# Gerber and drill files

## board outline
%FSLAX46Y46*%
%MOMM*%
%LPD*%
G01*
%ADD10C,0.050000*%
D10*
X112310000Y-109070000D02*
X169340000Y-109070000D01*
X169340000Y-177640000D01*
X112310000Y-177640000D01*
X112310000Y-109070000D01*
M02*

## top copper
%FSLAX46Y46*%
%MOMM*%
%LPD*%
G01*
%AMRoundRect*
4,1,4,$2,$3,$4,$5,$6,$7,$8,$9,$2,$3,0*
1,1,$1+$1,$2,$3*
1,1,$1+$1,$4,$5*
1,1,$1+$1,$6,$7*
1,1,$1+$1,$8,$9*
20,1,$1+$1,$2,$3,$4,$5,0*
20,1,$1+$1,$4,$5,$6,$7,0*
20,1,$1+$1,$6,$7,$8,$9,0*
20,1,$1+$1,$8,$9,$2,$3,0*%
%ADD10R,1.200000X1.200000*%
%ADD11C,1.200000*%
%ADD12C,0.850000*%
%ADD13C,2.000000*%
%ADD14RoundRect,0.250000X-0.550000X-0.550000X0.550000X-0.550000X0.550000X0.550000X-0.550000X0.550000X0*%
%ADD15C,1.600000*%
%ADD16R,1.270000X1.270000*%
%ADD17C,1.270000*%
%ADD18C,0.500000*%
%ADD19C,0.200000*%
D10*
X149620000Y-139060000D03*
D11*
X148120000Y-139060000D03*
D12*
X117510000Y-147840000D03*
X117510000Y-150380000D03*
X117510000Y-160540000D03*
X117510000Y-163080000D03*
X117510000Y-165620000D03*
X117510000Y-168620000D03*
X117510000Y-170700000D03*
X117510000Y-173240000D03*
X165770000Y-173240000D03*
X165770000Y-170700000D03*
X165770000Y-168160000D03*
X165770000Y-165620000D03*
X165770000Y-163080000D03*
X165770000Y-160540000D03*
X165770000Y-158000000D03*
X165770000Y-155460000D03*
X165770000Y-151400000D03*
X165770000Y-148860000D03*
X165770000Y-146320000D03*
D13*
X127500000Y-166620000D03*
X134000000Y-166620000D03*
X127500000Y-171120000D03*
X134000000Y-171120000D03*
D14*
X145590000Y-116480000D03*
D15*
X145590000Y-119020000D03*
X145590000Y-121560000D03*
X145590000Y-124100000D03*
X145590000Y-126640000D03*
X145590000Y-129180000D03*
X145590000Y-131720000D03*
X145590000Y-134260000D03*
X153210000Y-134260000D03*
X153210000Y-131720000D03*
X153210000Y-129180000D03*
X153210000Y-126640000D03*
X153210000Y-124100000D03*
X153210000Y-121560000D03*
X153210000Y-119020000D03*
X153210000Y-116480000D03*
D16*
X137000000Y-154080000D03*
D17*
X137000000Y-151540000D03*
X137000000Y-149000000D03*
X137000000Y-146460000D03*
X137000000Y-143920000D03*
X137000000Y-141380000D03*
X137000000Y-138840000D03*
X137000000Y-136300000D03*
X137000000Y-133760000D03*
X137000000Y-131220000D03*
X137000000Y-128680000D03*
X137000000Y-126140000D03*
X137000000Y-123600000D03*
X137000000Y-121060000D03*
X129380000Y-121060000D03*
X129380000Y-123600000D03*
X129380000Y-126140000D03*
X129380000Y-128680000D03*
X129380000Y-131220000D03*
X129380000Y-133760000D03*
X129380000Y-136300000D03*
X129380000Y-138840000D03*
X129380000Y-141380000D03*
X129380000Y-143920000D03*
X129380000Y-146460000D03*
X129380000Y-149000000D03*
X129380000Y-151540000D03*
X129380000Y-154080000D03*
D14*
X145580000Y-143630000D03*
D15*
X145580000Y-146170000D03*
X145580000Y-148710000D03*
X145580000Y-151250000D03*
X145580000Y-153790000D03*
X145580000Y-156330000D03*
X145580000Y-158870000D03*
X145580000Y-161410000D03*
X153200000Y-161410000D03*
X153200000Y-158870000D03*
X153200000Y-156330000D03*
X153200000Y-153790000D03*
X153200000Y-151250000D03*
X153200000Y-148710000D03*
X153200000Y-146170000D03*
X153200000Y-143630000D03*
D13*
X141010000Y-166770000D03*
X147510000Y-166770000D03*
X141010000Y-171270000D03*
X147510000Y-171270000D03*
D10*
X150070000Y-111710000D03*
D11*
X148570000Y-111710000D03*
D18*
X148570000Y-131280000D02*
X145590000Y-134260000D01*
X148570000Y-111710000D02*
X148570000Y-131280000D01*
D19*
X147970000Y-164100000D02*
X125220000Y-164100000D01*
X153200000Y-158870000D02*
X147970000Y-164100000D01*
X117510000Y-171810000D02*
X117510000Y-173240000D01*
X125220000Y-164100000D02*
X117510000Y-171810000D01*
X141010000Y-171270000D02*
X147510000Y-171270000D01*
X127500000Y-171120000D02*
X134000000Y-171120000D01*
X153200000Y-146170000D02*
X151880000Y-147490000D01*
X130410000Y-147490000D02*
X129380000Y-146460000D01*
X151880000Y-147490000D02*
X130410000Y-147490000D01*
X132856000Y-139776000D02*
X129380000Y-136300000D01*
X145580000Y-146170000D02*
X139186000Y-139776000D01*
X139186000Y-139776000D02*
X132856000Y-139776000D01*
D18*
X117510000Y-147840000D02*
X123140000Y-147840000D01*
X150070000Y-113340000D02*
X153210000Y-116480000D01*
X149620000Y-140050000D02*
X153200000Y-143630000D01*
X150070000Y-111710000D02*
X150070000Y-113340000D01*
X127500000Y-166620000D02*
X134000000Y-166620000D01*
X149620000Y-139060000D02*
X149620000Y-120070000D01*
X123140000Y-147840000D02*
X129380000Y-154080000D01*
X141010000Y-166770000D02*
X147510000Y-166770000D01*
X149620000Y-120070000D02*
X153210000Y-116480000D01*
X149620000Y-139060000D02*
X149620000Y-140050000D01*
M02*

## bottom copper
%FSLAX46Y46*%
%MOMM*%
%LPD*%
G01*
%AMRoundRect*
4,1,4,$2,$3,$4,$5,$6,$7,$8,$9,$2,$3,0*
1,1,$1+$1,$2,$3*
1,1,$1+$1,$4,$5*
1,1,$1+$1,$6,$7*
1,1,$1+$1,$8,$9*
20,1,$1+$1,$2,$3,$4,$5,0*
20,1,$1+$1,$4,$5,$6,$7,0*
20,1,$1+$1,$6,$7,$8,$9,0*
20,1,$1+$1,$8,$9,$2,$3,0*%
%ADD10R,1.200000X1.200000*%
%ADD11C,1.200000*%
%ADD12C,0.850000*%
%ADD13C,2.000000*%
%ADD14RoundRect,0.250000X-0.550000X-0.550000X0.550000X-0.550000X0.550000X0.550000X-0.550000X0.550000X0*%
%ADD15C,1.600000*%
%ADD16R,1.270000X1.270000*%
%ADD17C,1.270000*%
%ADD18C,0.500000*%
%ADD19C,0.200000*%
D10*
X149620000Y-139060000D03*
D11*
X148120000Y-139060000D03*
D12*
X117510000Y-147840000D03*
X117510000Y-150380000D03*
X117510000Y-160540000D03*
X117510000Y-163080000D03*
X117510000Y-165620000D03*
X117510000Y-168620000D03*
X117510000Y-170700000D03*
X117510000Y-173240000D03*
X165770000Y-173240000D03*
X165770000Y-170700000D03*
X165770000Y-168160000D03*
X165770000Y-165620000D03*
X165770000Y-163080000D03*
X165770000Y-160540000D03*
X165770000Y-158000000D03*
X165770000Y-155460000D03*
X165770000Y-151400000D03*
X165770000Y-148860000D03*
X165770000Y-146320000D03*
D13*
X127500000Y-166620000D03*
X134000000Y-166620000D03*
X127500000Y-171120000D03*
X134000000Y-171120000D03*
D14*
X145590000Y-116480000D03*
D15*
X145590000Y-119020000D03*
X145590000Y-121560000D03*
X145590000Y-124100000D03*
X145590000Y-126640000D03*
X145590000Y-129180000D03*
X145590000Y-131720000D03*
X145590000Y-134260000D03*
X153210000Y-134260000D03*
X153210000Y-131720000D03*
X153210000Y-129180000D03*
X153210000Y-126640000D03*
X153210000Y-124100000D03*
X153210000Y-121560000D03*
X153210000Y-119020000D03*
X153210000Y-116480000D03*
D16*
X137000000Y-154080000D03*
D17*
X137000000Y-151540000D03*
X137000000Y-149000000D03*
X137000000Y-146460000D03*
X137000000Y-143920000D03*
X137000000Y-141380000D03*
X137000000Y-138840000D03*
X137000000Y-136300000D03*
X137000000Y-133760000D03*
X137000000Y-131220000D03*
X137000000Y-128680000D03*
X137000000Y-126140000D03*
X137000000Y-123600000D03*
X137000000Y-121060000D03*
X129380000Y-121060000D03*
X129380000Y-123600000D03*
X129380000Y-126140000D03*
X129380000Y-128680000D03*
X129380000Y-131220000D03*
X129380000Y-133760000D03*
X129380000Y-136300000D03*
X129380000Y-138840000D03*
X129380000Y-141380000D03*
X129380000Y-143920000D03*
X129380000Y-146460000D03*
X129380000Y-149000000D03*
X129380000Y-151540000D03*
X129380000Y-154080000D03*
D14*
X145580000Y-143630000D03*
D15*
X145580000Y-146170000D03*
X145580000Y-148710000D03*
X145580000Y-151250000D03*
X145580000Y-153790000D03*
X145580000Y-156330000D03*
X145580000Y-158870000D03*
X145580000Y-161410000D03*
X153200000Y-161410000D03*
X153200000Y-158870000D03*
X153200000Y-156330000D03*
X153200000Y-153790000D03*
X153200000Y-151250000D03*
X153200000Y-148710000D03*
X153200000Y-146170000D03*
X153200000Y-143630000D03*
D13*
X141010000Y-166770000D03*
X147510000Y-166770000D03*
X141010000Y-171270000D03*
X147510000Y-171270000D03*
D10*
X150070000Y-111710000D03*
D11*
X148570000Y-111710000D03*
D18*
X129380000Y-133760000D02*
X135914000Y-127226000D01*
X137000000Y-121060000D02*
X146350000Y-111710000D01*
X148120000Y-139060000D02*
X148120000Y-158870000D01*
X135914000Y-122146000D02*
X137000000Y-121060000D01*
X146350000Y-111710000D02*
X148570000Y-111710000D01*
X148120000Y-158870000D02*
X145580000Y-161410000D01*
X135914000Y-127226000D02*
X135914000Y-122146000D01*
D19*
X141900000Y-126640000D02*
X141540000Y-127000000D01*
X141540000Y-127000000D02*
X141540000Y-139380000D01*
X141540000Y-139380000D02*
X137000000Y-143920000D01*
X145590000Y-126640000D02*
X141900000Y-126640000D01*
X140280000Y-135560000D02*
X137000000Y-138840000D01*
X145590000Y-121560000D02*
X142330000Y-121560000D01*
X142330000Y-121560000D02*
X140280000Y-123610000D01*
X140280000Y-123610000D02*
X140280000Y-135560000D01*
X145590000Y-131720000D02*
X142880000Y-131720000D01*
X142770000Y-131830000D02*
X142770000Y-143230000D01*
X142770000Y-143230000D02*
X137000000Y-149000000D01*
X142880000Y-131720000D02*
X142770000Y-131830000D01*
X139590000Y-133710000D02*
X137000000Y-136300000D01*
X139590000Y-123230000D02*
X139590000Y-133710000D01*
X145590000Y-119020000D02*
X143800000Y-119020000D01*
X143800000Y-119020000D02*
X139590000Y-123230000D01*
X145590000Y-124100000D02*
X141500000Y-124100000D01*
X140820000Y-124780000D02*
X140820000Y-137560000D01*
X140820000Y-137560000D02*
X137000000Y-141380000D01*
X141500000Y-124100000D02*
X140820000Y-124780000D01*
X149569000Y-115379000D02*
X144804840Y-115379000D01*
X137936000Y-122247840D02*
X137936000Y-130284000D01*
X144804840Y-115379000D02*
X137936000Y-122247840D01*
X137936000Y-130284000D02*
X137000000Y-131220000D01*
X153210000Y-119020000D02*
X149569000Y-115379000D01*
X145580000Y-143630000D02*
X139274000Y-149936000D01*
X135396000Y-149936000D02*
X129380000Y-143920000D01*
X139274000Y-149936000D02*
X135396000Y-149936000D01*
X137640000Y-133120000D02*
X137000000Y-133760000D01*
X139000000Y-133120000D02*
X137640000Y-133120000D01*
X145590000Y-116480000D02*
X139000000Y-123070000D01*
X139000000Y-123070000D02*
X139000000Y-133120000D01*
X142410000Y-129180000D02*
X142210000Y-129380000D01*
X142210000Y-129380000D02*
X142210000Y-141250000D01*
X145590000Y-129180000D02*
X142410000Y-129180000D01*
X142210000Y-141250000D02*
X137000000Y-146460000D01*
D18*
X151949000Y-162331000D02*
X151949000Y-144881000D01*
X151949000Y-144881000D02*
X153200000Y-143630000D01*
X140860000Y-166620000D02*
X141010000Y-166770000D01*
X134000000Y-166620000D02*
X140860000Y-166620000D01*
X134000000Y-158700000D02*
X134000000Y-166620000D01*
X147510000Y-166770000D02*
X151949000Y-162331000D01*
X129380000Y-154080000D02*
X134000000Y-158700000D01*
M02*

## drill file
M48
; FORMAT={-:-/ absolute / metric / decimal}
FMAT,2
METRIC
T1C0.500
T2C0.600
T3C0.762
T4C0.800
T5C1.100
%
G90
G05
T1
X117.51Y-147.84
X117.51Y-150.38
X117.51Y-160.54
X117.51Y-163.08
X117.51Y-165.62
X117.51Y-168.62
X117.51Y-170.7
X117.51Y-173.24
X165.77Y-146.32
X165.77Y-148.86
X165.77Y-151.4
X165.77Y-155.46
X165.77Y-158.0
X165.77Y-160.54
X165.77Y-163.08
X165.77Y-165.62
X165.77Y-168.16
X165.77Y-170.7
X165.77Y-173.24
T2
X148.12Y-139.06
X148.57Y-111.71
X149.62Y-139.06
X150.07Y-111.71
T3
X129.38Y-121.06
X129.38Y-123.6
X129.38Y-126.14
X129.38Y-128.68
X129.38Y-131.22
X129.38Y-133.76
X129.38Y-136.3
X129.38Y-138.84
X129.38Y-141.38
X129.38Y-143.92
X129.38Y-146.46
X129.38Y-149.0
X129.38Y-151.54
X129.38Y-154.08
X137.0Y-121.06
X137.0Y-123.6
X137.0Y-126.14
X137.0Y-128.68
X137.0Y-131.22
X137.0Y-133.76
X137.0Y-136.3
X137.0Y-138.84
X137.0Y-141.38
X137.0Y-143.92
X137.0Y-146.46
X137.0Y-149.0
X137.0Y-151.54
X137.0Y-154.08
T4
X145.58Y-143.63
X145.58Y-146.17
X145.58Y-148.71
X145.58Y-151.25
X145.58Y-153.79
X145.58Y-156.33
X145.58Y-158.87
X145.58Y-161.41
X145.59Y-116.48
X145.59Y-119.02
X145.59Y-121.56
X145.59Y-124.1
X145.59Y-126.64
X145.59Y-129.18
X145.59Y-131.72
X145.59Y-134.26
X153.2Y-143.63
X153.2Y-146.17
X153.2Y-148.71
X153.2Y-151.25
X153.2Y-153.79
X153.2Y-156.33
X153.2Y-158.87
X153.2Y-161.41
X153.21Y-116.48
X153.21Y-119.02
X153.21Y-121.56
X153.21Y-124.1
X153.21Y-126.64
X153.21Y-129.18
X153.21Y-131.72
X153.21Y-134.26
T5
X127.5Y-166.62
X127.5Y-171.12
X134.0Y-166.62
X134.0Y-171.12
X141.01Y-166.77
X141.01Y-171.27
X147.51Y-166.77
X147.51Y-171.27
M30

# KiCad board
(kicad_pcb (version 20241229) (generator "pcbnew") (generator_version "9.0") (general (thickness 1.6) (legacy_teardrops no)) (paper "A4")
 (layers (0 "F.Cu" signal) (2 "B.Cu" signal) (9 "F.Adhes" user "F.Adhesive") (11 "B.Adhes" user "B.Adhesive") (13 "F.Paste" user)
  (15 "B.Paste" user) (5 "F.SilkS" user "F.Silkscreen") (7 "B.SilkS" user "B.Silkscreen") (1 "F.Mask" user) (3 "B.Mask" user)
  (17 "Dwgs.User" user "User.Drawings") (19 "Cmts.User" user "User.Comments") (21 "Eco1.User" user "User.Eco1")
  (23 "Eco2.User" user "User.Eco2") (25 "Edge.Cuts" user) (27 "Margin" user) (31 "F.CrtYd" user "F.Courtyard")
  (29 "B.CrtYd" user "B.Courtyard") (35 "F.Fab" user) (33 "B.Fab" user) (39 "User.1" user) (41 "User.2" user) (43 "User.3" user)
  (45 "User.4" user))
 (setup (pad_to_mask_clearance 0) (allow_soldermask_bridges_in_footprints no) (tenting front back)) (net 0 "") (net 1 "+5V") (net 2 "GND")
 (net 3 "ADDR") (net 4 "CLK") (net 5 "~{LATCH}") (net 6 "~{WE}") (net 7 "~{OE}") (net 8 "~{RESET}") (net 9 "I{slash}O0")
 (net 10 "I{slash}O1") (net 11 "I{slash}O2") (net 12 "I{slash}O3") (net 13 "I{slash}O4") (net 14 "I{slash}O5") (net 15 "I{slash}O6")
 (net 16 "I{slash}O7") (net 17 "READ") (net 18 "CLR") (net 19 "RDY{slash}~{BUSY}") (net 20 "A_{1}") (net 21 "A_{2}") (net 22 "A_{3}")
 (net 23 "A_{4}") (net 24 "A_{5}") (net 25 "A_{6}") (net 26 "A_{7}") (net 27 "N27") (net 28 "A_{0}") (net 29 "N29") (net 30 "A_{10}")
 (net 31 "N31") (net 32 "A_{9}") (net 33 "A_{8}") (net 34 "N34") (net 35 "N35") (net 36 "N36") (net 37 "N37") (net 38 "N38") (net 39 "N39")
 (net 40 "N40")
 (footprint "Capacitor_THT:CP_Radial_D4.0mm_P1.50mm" (layer "F.Cu") (at 149.62 139.06 180)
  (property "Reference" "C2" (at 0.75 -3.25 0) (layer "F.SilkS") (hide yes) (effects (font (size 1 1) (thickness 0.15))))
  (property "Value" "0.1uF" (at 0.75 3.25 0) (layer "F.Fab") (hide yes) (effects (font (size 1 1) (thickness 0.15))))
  (pad "1" thru_hole rect (at 0 0 180) (size 1.2 1.2) (drill 0.6) (layers "*.Cu" "*.Mask") (remove_unused_layers no) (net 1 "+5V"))
  (pad "2" thru_hole circle (at 1.5 0 180) (size 1.2 1.2) (drill 0.6) (layers "*.Cu" "*.Mask") (remove_unused_layers no) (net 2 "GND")))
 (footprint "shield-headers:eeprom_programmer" (layer "F.Cu") (at 140.37 163.08)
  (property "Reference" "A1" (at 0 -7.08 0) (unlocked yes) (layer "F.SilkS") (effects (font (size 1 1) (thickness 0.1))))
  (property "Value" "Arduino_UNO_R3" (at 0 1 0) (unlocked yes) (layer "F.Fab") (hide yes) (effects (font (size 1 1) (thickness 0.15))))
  (pad "5" thru_hole circle (at -22.86 -15.24) (size 0.85 0.85) (drill 0.5) (layers "*.Cu" "*.Mask") (remove_unused_layers no) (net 1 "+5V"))
  (pad "6" thru_hole circle (at -22.86 -12.7) (size 0.85 0.85) (drill 0.5) (layers "*.Cu" "*.Mask") (remove_unused_layers no) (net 2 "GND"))
  (pad "9" thru_hole circle (at -22.86 -2.54) (size 0.85 0.85) (drill 0.5) (layers "*.Cu" "*.Mask") (remove_unused_layers no) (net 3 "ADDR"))
  (pad "10" thru_hole circle (at -22.86 0) (size 0.85 0.85) (drill 0.5) (layers "*.Cu" "*.Mask") (remove_unused_layers no) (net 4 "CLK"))
  (pad "11" thru_hole circle (at -22.86 2.54) (size 0.85 0.85) (drill 0.5) (layers "*.Cu" "*.Mask") (remove_unused_layers no)
   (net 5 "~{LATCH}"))
  (pad "12" thru_hole circle (at -22.86 5.54) (size 0.85 0.85) (drill 0.5) (layers "*.Cu" "*.Mask") (remove_unused_layers no)
   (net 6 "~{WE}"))
  (pad "13" thru_hole circle (at -22.86 7.62) (size 0.85 0.85) (drill 0.5) (layers "*.Cu" "*.Mask") (remove_unused_layers no)
   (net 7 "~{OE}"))
  (pad "14" thru_hole circle (at -22.86 10.16) (size 0.85 0.85) (drill 0.5) (layers "*.Cu" "*.Mask") (remove_unused_layers no)
   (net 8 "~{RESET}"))
  (pad "15" thru_hole circle (at 25.4 10.16) (size 0.85 0.85) (drill 0.5) (layers "*.Cu" "*.Mask") (remove_unused_layers no)
   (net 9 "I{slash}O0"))
  (pad "16" thru_hole circle (at 25.4 7.62) (size 0.85 0.85) (drill 0.5) (layers "*.Cu" "*.Mask") (remove_unused_layers no)
   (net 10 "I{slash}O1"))
  (pad "17" thru_hole circle (at 25.4 5.08) (size 0.85 0.85) (drill 0.5) (layers "*.Cu" "*.Mask") (remove_unused_layers no)
   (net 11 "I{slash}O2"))
  (pad "18" thru_hole circle (at 25.4 2.54) (size 0.85 0.85) (drill 0.5) (layers "*.Cu" "*.Mask") (remove_unused_layers no)
   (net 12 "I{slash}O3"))
  (pad "19" thru_hole circle (at 25.4 0) (size 0.85 0.85) (drill 0.5) (layers "*.Cu" "*.Mask") (remove_unused_layers no)
   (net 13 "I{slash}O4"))
  (pad "20" thru_hole circle (at 25.4 -2.54) (size 0.85 0.85) (drill 0.5) (layers "*.Cu" "*.Mask") (remove_unused_layers no)
   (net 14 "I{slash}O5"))
  (pad "21" thru_hole circle (at 25.4 -5.08) (size 0.85 0.85) (drill 0.5) (layers "*.Cu" "*.Mask") (remove_unused_layers no)
   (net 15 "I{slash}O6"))
  (pad "22" thru_hole circle (at 25.4 -7.62) (size 0.85 0.85) (drill 0.5) (layers "*.Cu" "*.Mask") (remove_unused_layers no)
   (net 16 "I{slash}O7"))
  (pad "23" thru_hole circle (at 25.4 -11.68) (size 0.85 0.85) (drill 0.5) (layers "*.Cu" "*.Mask") (remove_unused_layers no)
   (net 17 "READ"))
  (pad "24" thru_hole circle (at 25.4 -14.22) (size 0.85 0.85) (drill 0.5) (layers "*.Cu" "*.Mask") (remove_unused_layers no) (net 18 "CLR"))
  (pad "25" thru_hole circle (at 25.4 -16.76) (size 0.85 0.85) (drill 0.5) (layers "*.Cu" "*.Mask") (remove_unused_layers no)
   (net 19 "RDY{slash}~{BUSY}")))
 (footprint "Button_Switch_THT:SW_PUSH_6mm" (layer "F.Cu") (at 127.5 166.62)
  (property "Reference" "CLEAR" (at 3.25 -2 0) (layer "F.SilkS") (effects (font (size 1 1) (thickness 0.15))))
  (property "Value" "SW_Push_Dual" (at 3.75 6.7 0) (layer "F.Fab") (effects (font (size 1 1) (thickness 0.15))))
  (pad "1" thru_hole circle (at 0 0 90) (size 2 2) (drill 1.1) (layers "*.Cu" "*.Mask") (remove_unused_layers no) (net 1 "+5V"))
  (pad "1" thru_hole circle (at 6.5 0 90) (size 2 2) (drill 1.1) (layers "*.Cu" "*.Mask") (remove_unused_layers no) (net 1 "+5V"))
  (pad "2" thru_hole circle (at 0 4.5 90) (size 2 2) (drill 1.1) (layers "*.Cu" "*.Mask") (remove_unused_layers no) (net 18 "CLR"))
  (pad "2" thru_hole circle (at 6.5 4.5 90) (size 2 2) (drill 1.1) (layers "*.Cu" "*.Mask") (remove_unused_layers no) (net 18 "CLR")))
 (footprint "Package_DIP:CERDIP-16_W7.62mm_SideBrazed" (layer "F.Cu") (at 145.59 116.48)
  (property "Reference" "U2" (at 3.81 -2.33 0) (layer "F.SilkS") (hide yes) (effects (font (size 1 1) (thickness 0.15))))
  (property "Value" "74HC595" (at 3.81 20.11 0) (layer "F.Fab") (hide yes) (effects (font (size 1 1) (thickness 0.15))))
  (pad "1" thru_hole roundrect (at 0 0) (size 1.6 1.6) (drill 0.8) (layers "*.Cu" "*.Mask") (remove_unused_layers no)
   (roundrect_rratio 0.15625) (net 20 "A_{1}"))
  (pad "2" thru_hole circle (at 0 2.54) (size 1.6 1.6) (drill 0.8) (layers "*.Cu" "*.Mask") (remove_unused_layers no) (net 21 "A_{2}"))
  (pad "3" thru_hole circle (at 0 5.08) (size 1.6 1.6) (drill 0.8) (layers "*.Cu" "*.Mask") (remove_unused_layers no) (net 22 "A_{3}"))
  (pad "4" thru_hole circle (at 0 7.62) (size 1.6 1.6) (drill 0.8) (layers "*.Cu" "*.Mask") (remove_unused_layers no) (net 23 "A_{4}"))
  (pad "5" thru_hole circle (at 0 10.16) (size 1.6 1.6) (drill 0.8) (layers "*.Cu" "*.Mask") (remove_unused_layers no) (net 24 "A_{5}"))
  (pad "6" thru_hole circle (at 0 12.7) (size 1.6 1.6) (drill 0.8) (layers "*.Cu" "*.Mask") (remove_unused_layers no) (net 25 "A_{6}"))
  (pad "7" thru_hole circle (at 0 15.24) (size 1.6 1.6) (drill 0.8) (layers "*.Cu" "*.Mask") (remove_unused_layers no) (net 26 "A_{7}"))
  (pad "8" thru_hole circle (at 0 17.78) (size 1.6 1.6) (drill 0.8) (layers "*.Cu" "*.Mask") (remove_unused_layers no) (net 2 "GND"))
  (pad "9" thru_hole circle (at 7.62 17.78) (size 1.6 1.6) (drill 0.8) (layers "*.Cu" "*.Mask") (remove_unused_layers no) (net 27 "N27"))
  (pad "10" thru_hole circle (at 7.62 15.24) (size 1.6 1.6) (drill 0.8) (layers "*.Cu" "*.Mask") (remove_unused_layers no)
   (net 8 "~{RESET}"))
  (pad "11" thru_hole circle (at 7.62 12.7) (size 1.6 1.6) (drill 0.8) (layers "*.Cu" "*.Mask") (remove_unused_layers no) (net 4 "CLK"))
  (pad "12" thru_hole circle (at 7.62 10.16) (size 1.6 1.6) (drill 0.8) (layers "*.Cu" "*.Mask") (remove_unused_layers no) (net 4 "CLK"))
  (pad "13" thru_hole circle (at 7.62 7.62) (size 1.6 1.6) (drill 0.8) (layers "*.Cu" "*.Mask") (remove_unused_layers no) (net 5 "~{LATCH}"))
  (pad "14" thru_hole circle (at 7.62 5.08) (size 1.6 1.6) (drill 0.8) (layers "*.Cu" "*.Mask") (remove_unused_layers no) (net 3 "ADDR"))
  (pad "15" thru_hole circle (at 7.62 2.54) (size 1.6 1.6) (drill 0.8) (layers "*.Cu" "*.Mask") (remove_unused_layers no) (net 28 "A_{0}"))
  (pad "16" thru_hole circle (at 7.62 0) (size 1.6 1.6) (drill 0.8) (layers "*.Cu" "*.Mask") (remove_unused_layers no) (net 1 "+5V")))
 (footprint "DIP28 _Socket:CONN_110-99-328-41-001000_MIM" (layer "F.Cu") (at 137 154.08 180)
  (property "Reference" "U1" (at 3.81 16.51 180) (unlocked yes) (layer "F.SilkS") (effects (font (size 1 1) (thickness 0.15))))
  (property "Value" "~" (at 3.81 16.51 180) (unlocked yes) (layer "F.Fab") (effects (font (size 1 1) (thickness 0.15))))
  (pad "1" thru_hole rect (at 0 0 180) (size 1.27 1.27) (drill 0.762) (layers "*.Cu" "*.Mask") (remove_unused_layers no)
   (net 19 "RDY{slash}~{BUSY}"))
  (pad "2" thru_hole circle (at 0 2.54 180) (size 1.27 1.27) (drill 0.762) (layers "*.Cu" "*.Mask") (remove_unused_layers no) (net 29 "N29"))
  (pad "3" thru_hole circle (at 0 5.08 180) (size 1.27 1.27) (drill 0.762) (layers "*.Cu" "*.Mask") (remove_unused_layers no)
   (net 26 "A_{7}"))
  (pad "4" thru_hole circle (at 0 7.62 180) (size 1.27 1.27) (drill 0.762) (layers "*.Cu" "*.Mask") (remove_unused_layers no)
   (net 25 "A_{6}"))
  (pad "5" thru_hole circle (at 0 10.16 180) (size 1.27 1.27) (drill 0.762) (layers "*.Cu" "*.Mask") (remove_unused_layers no)
   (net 24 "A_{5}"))
  (pad "6" thru_hole circle (at 0 12.7 180) (size 1.27 1.27) (drill 0.762) (layers "*.Cu" "*.Mask") (remove_unused_layers no)
   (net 23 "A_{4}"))
  (pad "7" thru_hole circle (at 0 15.24 180) (size 1.27 1.27) (drill 0.762) (layers "*.Cu" "*.Mask") (remove_unused_layers no)
   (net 22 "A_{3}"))
  (pad "8" thru_hole circle (at 0 17.78 180) (size 1.27 1.27) (drill 0.762) (layers "*.Cu" "*.Mask") (remove_unused_layers no)
   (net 21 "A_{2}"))
  (pad "9" thru_hole circle (at 0 20.32 180) (size 1.27 1.27) (drill 0.762) (layers "*.Cu" "*.Mask") (remove_unused_layers no)
   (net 20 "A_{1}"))
  (pad "10" thru_hole circle (at 0 22.86 180) (size 1.27 1.27) (drill 0.762) (layers "*.Cu" "*.Mask") (remove_unused_layers no)
   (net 28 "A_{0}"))
  (pad "11" thru_hole circle (at 0 25.4 180) (size 1.27 1.27) (drill 0.762) (layers "*.Cu" "*.Mask") (remove_unused_layers no)
   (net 9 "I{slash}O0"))
  (pad "12" thru_hole circle (at 0 27.94 180) (size 1.27 1.27) (drill 0.762) (layers "*.Cu" "*.Mask") (remove_unused_layers no)
   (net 10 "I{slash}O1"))
  (pad "13" thru_hole circle (at 0 30.48 180) (size 1.27 1.27) (drill 0.762) (layers "*.Cu" "*.Mask") (remove_unused_layers no)
   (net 11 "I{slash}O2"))
  (pad "14" thru_hole circle (at 0 33.02 180) (size 1.27 1.27) (drill 0.762) (layers "*.Cu" "*.Mask") (remove_unused_layers no)
   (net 2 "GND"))
  (pad "15" thru_hole circle (at 7.62 33.02 180) (size 1.27 1.27) (drill 0.762) (layers "*.Cu" "*.Mask") (remove_unused_layers no)
   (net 12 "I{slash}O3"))
  (pad "16" thru_hole circle (at 7.62 30.48 180) (size 1.27 1.27) (drill 0.762) (layers "*.Cu" "*.Mask") (remove_unused_layers no)
   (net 13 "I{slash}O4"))
  (pad "17" thru_hole circle (at 7.62 27.94 180) (size 1.27 1.27) (drill 0.762) (layers "*.Cu" "*.Mask") (remove_unused_layers no)
   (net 14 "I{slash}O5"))
  (pad "18" thru_hole circle (at 7.62 25.4 180) (size 1.27 1.27) (drill 0.762) (layers "*.Cu" "*.Mask") (remove_unused_layers no)
   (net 15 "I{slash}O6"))
  (pad "19" thru_hole circle (at 7.62 22.86 180) (size 1.27 1.27) (drill 0.762) (layers "*.Cu" "*.Mask") (remove_unused_layers no)
   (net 16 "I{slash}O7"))
  (pad "20" thru_hole circle (at 7.62 20.32 180) (size 1.27 1.27) (drill 0.762) (layers "*.Cu" "*.Mask") (remove_unused_layers no)
   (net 2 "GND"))
  (pad "21" thru_hole circle (at 7.62 17.78 180) (size 1.27 1.27) (drill 0.762) (layers "*.Cu" "*.Mask") (remove_unused_layers no)
   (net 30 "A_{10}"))
  (pad "22" thru_hole circle (at 7.62 15.24 180) (size 1.27 1.27) (drill 0.762) (layers "*.Cu" "*.Mask") (remove_unused_layers no)
   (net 7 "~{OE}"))
  (pad "23" thru_hole circle (at 7.62 12.7 180) (size 1.27 1.27) (drill 0.762) (layers "*.Cu" "*.Mask") (remove_unused_layers no)
   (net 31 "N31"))
  (pad "24" thru_hole circle (at 7.62 10.16 180) (size 1.27 1.27) (drill 0.762) (layers "*.Cu" "*.Mask") (remove_unused_layers no)
   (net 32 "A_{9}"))
  (pad "25" thru_hole circle (at 7.62 7.62 180) (size 1.27 1.27) (drill 0.762) (layers "*.Cu" "*.Mask") (remove_unused_layers no)
   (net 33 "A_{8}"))
  (pad "26" thru_hole circle (at 7.62 5.08 180) (size 1.27 1.27) (drill 0.762) (layers "*.Cu" "*.Mask") (remove_unused_layers no)
   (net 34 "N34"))
  (pad "27" thru_hole circle (at 7.62 2.54 180) (size 1.27 1.27) (drill 0.762) (layers "*.Cu" "*.Mask") (remove_unused_layers no)
   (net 6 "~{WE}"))
  (pad "28" thru_hole circle (at 7.62 0 180) (size 1.27 1.27) (drill 0.762) (layers "*.Cu" "*.Mask") (remove_unused_layers no) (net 1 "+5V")))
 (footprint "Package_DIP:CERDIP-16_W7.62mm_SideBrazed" (layer "F.Cu") (at 145.58 143.63)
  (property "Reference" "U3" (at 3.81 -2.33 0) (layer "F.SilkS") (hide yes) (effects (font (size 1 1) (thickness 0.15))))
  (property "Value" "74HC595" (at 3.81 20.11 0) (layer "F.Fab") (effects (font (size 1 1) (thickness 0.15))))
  (pad "1" thru_hole roundrect (at 0 0) (size 1.6 1.6) (drill 0.8) (layers "*.Cu" "*.Mask") (remove_unused_layers no)
   (roundrect_rratio 0.15625) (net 32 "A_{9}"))
  (pad "2" thru_hole circle (at 0 2.54) (size 1.6 1.6) (drill 0.8) (layers "*.Cu" "*.Mask") (remove_unused_layers no) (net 30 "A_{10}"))
  (pad "3" thru_hole circle (at 0 5.08) (size 1.6 1.6) (drill 0.8) (layers "*.Cu" "*.Mask") (remove_unused_layers no) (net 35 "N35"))
  (pad "4" thru_hole circle (at 0 7.62) (size 1.6 1.6) (drill 0.8) (layers "*.Cu" "*.Mask") (remove_unused_layers no) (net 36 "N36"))
  (pad "5" thru_hole circle (at 0 10.16) (size 1.6 1.6) (drill 0.8) (layers "*.Cu" "*.Mask") (remove_unused_layers no) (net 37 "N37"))
  (pad "6" thru_hole circle (at 0 12.7) (size 1.6 1.6) (drill 0.8) (layers "*.Cu" "*.Mask") (remove_unused_layers no) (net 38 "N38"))
  (pad "7" thru_hole circle (at 0 15.24) (size 1.6 1.6) (drill 0.8) (layers "*.Cu" "*.Mask") (remove_unused_layers no) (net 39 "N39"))
  (pad "8" thru_hole circle (at 0 17.78) (size 1.6 1.6) (drill 0.8) (layers "*.Cu" "*.Mask") (remove_unused_layers no) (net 2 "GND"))
  (pad "9" thru_hole circle (at 7.62 17.78) (size 1.6 1.6) (drill 0.8) (layers "*.Cu" "*.Mask") (remove_unused_layers no) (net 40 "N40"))
  (pad "10" thru_hole circle (at 7.62 15.24) (size 1.6 1.6) (drill 0.8) (layers "*.Cu" "*.Mask") (remove_unused_layers no)
   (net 8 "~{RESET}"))
  (pad "11" thru_hole circle (at 7.62 12.7) (size 1.6 1.6) (drill 0.8) (layers "*.Cu" "*.Mask") (remove_unused_layers no) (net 4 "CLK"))
  (pad "12" thru_hole circle (at 7.62 10.16) (size 1.6 1.6) (drill 0.8) (layers "*.Cu" "*.Mask") (remove_unused_layers no) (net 4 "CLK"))
  (pad "13" thru_hole circle (at 7.62 7.62) (size 1.6 1.6) (drill 0.8) (layers "*.Cu" "*.Mask") (remove_unused_layers no) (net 5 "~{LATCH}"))
  (pad "14" thru_hole circle (at 7.62 5.08) (size 1.6 1.6) (drill 0.8) (layers "*.Cu" "*.Mask") (remove_unused_layers no) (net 27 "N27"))
  (pad "15" thru_hole circle (at 7.62 2.54) (size 1.6 1.6) (drill 0.8) (layers "*.Cu" "*.Mask") (remove_unused_layers no) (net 33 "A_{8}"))
  (pad "16" thru_hole circle (at 7.62 0) (size 1.6 1.6) (drill 0.8) (layers "*.Cu" "*.Mask") (remove_unused_layers no) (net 1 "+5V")))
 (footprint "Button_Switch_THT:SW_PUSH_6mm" (layer "F.Cu") (at 141.01 166.77)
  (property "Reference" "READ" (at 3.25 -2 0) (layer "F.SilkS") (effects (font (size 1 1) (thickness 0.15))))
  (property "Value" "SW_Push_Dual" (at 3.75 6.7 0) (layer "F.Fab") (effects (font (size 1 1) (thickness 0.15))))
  (pad "1" thru_hole circle (at 0 0 90) (size 2 2) (drill 1.1) (layers "*.Cu" "*.Mask") (remove_unused_layers no) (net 1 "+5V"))
  (pad "1" thru_hole circle (at 6.5 0 90) (size 2 2) (drill 1.1) (layers "*.Cu" "*.Mask") (remove_unused_layers no) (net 1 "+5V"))
  (pad "2" thru_hole circle (at 0 4.5 90) (size 2 2) (drill 1.1) (layers "*.Cu" "*.Mask") (remove_unused_layers no) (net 17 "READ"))
  (pad "2" thru_hole circle (at 6.5 4.5 90) (size 2 2) (drill 1.1) (layers "*.Cu" "*.Mask") (remove_unused_layers no) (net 17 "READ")))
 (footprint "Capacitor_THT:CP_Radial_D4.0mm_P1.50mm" (layer "F.Cu") (at 150.07 111.71 180)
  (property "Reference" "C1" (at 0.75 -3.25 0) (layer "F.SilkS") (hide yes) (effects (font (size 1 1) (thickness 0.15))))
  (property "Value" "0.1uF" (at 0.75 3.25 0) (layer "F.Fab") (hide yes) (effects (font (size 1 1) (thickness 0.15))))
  (pad "1" thru_hole rect (at 0 0 180) (size 1.2 1.2) (drill 0.6) (layers "*.Cu" "*.Mask") (remove_unused_layers no) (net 1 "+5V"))
  (pad "2" thru_hole circle (at 1.5 0 180) (size 1.2 1.2) (drill 0.6) (layers "*.Cu" "*.Mask") (remove_unused_layers no) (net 2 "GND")))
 (gr_rect (start 112.31 109.07) (end 169.34 177.64) (stroke (width 0.05) (type default)) (fill no) (layer "Edge.Cuts"))
 (segment (start 148.57 131.28) (end 145.59 134.26) (width 0.5) (layer "F.Cu") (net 2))
 (segment (start 148.57 111.71) (end 148.57 131.28) (width 0.5) (layer "F.Cu") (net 2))
 (segment (start 129.38 133.76) (end 135.914 127.226) (width 0.5) (layer "B.Cu") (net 2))
 (segment (start 137 121.06) (end 146.35 111.71) (width 0.5) (layer "B.Cu") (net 2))
 (segment (start 148.12 139.06) (end 148.12 158.87) (width 0.5) (layer "B.Cu") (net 2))
 (segment (start 135.914 122.146) (end 137 121.06) (width 0.5) (layer "B.Cu") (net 2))
 (segment (start 146.35 111.71) (end 148.57 111.71) (width 0.5) (layer "B.Cu") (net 2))
 (segment (start 148.12 158.87) (end 145.58 161.41) (width 0.5) (layer "B.Cu") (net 2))
 (segment (start 135.914 127.226) (end 135.914 122.146) (width 0.5) (layer "B.Cu") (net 2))
 (segment (start 147.97 164.1) (end 125.22 164.1) (width 0.2) (layer "F.Cu") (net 8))
 (segment (start 153.2 158.87) (end 147.97 164.1) (width 0.2) (layer "F.Cu") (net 8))
 (segment (start 117.51 171.81) (end 117.51 173.24) (width 0.2) (layer "F.Cu") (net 8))
 (segment (start 125.22 164.1) (end 117.51 171.81) (width 0.2) (layer "F.Cu") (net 8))
 (segment (start 141.01 171.27) (end 147.51 171.27) (width 0.2) (layer "F.Cu") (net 17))
 (segment (start 127.5 171.12) (end 134 171.12) (width 0.2) (layer "F.Cu") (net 18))
 (segment (start 141.9 126.64) (end 141.54 127) (width 0.2) (layer "B.Cu") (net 24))
 (segment (start 141.54 127) (end 141.54 139.38) (width 0.2) (layer "B.Cu") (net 24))
 (segment (start 141.54 139.38) (end 137 143.92) (width 0.2) (layer "B.Cu") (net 24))
 (segment (start 145.59 126.64) (end 141.9 126.64) (width 0.2) (layer "B.Cu") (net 24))
 (segment (start 140.28 135.56) (end 137 138.84) (width 0.2) (layer "B.Cu") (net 22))
 (segment (start 145.59 121.56) (end 142.33 121.56) (width 0.2) (layer "B.Cu") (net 22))
 (segment (start 142.33 121.56) (end 140.28 123.61) (width 0.2) (layer "B.Cu") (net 22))
 (segment (start 140.28 123.61) (end 140.28 135.56) (width 0.2) (layer "B.Cu") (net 22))
 (segment (start 145.59 131.72) (end 142.88 131.72) (width 0.2) (layer "B.Cu") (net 26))
 (segment (start 142.77 131.83) (end 142.77 143.23) (width 0.2) (layer "B.Cu") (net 26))
 (segment (start 142.77 143.23) (end 137 149) (width 0.2) (layer "B.Cu") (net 26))
 (segment (start 142.88 131.72) (end 142.77 131.83) (width 0.2) (layer "B.Cu") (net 26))
 (segment (start 139.59 133.71) (end 137 136.3) (width 0.2) (layer "B.Cu") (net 21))
 (segment (start 139.59 123.23) (end 139.59 133.71) (width 0.2) (layer "B.Cu") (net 21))
 (segment (start 145.59 119.02) (end 143.8 119.02) (width 0.2) (layer "B.Cu") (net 21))
 (segment (start 143.8 119.02) (end 139.59 123.23) (width 0.2) (layer "B.Cu") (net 21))
 (segment (start 153.2 146.17) (end 151.88 147.49) (width 0.2) (layer "F.Cu") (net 33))
 (segment (start 130.41 147.49) (end 129.38 146.46) (width 0.2) (layer "F.Cu") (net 33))
 (segment (start 151.88 147.49) (end 130.41 147.49) (width 0.2) (layer "F.Cu") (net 33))
 (segment (start 145.59 124.1) (end 141.5 124.1) (width 0.2) (layer "B.Cu") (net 23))
 (segment (start 140.82 124.78) (end 140.82 137.56) (width 0.2) (layer "B.Cu") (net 23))
 (segment (start 140.82 137.56) (end 137 141.38) (width 0.2) (layer "B.Cu") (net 23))
 (segment (start 141.5 124.1) (end 140.82 124.78) (width 0.2) (layer "B.Cu") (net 23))
 (segment (start 149.569 115.379) (end 144.80484 115.379) (width 0.2) (layer "B.Cu") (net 28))
 (segment (start 137.936 122.24784) (end 137.936 130.284) (width 0.2) (layer "B.Cu") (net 28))
 (segment (start 144.80484 115.379) (end 137.936 122.24784) (width 0.2) (layer "B.Cu") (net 28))
 (segment (start 137.936 130.284) (end 137 131.22) (width 0.2) (layer "B.Cu") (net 28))
 (segment (start 153.21 119.02) (end 149.569 115.379) (width 0.2) (layer "B.Cu") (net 28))
 (segment (start 145.58 143.63) (end 139.274 149.936) (width 0.2) (layer "B.Cu") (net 32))
 (segment (start 135.396 149.936) (end 129.38 143.92) (width 0.2) (layer "B.Cu") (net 32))
 (segment (start 139.274 149.936) (end 135.396 149.936) (width 0.2) (layer "B.Cu") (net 32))
 (segment (start 132.856 139.776) (end 129.38 136.3) (width 0.2) (layer "F.Cu") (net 30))
 (segment (start 145.58 146.17) (end 139.186 139.776) (width 0.2) (layer "F.Cu") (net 30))
 (segment (start 139.186 139.776) (end 132.856 139.776) (width 0.2) (layer "F.Cu") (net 30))
 (segment (start 137.64 133.12) (end 137 133.76) (width 0.2) (layer "B.Cu") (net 20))
 (segment (start 139 133.12) (end 137.64 133.12) (width 0.2) (layer "B.Cu") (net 20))
 (segment (start 145.59 116.48) (end 139 123.07) (width 0.2) (layer "B.Cu") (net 20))
 (segment (start 139 123.07) (end 139 133.12) (width 0.2) (layer "B.Cu") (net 20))
 (segment (start 142.41 129.18) (end 142.21 129.38) (width 0.2) (layer "B.Cu") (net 25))
 (segment (start 142.21 129.38) (end 142.21 141.25) (width 0.2) (layer "B.Cu") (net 25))
 (segment (start 145.59 129.18) (end 142.41 129.18) (width 0.2) (layer "B.Cu") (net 25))
 (segment (start 142.21 141.25) (end 137 146.46) (width 0.2) (layer "B.Cu") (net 25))
 (segment (start 117.51 147.84) (end 123.14 147.84) (width 0.5) (layer "F.Cu") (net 1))
 (segment (start 150.07 113.34) (end 153.21 116.48) (width 0.5) (layer "F.Cu") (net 1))
 (segment (start 149.62 140.05) (end 153.2 143.63) (width 0.5) (layer "F.Cu") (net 1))
 (segment (start 150.07 111.71) (end 150.07 113.34) (width 0.5) (layer "F.Cu") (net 1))
 (segment (start 127.5 166.62) (end 134 166.62) (width 0.5) (layer "F.Cu") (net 1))
 (segment (start 149.62 139.06) (end 149.62 120.07) (width 0.5) (layer "F.Cu") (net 1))
 (segment (start 123.14 147.84) (end 129.38 154.08) (width 0.5) (layer "F.Cu") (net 1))
 (segment (start 141.01 166.77) (end 147.51 166.77) (width 0.5) (layer "F.Cu") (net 1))
 (segment (start 149.62 120.07) (end 153.21 116.48) (width 0.5) (layer "F.Cu") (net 1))
 (segment (start 149.62 139.06) (end 149.62 140.05) (width 0.5) (layer "F.Cu") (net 1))
 (segment (start 151.949 162.331) (end 151.949 144.881) (width 0.5) (layer "B.Cu") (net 1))
 (segment (start 151.949 144.881) (end 153.2 143.63) (width 0.5) (layer "B.Cu") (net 1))
 (segment (start 140.86 166.62) (end 141.01 166.77) (width 0.5) (layer "B.Cu") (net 1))
 (segment (start 134 166.62) (end 140.86 166.62) (width 0.5) (layer "B.Cu") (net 1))
 (segment (start 134 158.7) (end 134 166.62) (width 0.5) (layer "B.Cu") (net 1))
 (segment (start 147.51 166.77) (end 151.949 162.331) (width 0.5) (layer "B.Cu") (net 1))
 (segment (start 129.38 154.08) (end 134 158.7) (width 0.5) (layer "B.Cu") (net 1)))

